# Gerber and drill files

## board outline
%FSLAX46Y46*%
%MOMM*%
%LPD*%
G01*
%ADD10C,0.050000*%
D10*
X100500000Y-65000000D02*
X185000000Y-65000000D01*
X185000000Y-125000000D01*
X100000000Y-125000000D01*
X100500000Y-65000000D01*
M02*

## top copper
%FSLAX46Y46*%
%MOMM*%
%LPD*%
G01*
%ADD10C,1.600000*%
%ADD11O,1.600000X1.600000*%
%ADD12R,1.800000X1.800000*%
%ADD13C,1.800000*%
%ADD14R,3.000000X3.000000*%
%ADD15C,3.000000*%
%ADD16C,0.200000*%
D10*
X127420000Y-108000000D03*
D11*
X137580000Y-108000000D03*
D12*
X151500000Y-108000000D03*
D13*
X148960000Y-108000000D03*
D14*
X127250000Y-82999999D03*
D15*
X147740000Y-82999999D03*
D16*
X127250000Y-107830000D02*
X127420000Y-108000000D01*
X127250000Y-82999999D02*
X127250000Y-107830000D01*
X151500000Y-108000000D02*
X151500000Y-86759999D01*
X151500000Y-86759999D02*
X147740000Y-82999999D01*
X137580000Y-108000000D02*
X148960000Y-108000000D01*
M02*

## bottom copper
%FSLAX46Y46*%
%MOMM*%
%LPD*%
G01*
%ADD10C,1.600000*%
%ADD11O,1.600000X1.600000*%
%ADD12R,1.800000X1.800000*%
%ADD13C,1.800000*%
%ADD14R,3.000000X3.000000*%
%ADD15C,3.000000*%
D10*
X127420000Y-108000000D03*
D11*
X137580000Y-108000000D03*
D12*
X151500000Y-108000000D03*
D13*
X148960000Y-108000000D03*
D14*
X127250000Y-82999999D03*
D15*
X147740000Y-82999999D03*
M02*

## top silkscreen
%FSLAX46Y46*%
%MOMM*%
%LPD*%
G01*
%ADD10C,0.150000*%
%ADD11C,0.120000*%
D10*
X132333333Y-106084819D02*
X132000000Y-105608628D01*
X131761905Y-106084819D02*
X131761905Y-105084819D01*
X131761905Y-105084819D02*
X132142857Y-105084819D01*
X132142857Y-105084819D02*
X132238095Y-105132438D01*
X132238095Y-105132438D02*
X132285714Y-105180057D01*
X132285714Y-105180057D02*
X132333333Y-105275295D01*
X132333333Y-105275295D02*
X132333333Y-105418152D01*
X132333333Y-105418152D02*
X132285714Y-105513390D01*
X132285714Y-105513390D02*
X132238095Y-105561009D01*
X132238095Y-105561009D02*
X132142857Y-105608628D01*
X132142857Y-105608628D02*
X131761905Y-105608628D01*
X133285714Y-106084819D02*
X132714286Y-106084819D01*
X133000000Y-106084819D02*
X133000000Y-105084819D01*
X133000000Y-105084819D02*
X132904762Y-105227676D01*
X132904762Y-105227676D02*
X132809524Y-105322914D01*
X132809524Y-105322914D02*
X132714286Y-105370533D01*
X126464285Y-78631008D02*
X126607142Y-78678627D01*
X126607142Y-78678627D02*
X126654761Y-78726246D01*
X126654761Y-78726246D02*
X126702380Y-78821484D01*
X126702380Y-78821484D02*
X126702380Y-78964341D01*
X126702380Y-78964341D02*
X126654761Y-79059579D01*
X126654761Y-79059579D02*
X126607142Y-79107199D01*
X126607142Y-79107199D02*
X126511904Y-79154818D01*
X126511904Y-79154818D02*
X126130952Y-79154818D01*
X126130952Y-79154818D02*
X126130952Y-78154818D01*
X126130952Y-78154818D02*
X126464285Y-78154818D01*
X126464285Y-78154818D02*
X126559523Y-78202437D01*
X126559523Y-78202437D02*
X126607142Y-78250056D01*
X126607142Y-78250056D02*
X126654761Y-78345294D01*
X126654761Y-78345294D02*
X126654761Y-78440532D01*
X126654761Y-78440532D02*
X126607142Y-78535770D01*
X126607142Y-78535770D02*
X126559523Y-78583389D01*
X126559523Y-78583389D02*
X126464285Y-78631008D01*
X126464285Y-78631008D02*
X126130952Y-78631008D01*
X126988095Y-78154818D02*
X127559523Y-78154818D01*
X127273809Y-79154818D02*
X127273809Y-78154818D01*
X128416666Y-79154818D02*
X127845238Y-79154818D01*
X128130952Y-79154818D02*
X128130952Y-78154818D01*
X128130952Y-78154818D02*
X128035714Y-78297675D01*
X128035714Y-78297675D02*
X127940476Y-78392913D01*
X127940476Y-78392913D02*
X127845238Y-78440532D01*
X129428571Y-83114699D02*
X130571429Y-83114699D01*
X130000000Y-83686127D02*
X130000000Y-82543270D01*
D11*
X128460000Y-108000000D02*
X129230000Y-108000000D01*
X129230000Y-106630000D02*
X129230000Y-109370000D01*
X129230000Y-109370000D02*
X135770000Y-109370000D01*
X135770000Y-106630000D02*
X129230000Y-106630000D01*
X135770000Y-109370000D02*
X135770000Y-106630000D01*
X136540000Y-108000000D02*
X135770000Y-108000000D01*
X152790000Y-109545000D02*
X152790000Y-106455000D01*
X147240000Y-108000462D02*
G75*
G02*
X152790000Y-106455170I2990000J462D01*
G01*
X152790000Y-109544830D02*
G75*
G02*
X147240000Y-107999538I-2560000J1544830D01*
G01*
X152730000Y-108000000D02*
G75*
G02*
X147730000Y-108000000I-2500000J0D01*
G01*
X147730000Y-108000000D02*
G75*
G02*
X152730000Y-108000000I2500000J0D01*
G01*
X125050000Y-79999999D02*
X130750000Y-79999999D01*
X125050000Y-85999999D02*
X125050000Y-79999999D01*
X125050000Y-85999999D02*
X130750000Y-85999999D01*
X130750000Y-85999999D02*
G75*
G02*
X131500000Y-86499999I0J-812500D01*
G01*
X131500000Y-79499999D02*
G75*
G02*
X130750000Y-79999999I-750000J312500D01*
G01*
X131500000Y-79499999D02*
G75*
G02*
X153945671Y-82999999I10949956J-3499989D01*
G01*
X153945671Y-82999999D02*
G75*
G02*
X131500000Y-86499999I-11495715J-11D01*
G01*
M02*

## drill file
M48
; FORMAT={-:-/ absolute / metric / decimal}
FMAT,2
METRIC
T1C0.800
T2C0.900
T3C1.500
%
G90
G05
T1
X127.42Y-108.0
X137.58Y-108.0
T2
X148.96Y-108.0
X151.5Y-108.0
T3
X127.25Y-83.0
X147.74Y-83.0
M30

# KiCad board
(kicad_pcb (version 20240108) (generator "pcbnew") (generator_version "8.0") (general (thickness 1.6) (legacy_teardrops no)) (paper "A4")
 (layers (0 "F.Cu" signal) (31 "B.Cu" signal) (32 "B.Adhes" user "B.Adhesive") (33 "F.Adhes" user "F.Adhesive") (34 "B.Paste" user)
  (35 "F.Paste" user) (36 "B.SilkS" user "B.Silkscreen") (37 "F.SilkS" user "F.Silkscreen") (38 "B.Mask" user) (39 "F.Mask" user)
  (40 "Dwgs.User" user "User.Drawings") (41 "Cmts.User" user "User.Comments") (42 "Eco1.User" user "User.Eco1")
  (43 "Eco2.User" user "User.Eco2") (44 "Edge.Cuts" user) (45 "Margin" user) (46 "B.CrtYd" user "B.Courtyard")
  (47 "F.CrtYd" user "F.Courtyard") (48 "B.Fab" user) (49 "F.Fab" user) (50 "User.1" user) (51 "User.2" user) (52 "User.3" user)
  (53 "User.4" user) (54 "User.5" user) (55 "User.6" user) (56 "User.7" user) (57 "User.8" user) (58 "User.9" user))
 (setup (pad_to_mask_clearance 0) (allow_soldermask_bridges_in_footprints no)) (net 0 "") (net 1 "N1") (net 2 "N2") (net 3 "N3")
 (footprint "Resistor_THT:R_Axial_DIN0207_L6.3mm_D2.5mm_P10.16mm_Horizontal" (layer "F.Cu") (at 127.42 108)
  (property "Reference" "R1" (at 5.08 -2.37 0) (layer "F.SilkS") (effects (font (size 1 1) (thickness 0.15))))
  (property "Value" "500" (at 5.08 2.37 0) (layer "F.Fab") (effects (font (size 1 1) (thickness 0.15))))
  (fp_line (start 1.04 0) (end 1.81 0) (stroke (width 0.12) (type solid)) (layer "F.SilkS"))
  (fp_line (start 1.81 -1.37) (end 1.81 1.37) (stroke (width 0.12) (type solid)) (layer "F.SilkS"))
  (fp_line (start 1.81 1.37) (end 8.35 1.37) (stroke (width 0.12) (type solid)) (layer "F.SilkS"))
  (fp_line (start 8.35 -1.37) (end 1.81 -1.37) (stroke (width 0.12) (type solid)) (layer "F.SilkS"))
  (fp_line (start 8.35 1.37) (end 8.35 -1.37) (stroke (width 0.12) (type solid)) (layer "F.SilkS"))
  (fp_line (start 9.12 0) (end 8.35 0) (stroke (width 0.12) (type solid)) (layer "F.SilkS"))
  (pad "1" thru_hole circle (at 0 0) (size 1.6 1.6) (drill 0.8) (layers "*.Cu" "*.Mask") (remove_unused_layers no) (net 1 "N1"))
  (pad "2" thru_hole oval (at 10.16 0) (size 1.6 1.6) (drill 0.8) (layers "*.Cu" "*.Mask") (remove_unused_layers no) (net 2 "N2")))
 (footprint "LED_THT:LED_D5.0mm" (layer "F.Cu") (at 151.5 108 180)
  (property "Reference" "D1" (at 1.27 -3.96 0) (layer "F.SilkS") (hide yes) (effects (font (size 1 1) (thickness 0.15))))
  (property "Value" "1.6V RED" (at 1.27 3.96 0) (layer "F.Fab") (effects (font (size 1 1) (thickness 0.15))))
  (fp_line (start -1.29 -1.545) (end -1.29 1.545) (stroke (width 0.12) (type solid)) (layer "F.SilkS"))
  (fp_arc (start 4.26 -0.000462) (mid 2.072002 2.880433) (end -1.29 1.54483) (stroke (width 0.12) (type solid)) (layer "F.SilkS"))
  (fp_arc (start -1.29 -1.54483) (mid 2.072002 -2.880433) (end 4.26 0.000462) (stroke (width 0.12) (type solid)) (layer "F.SilkS"))
  (fp_circle (center 1.27 0) (end 3.77 0) (stroke (width 0.12) (type solid)) (fill none) (layer "F.SilkS"))
  (pad "1" thru_hole rect (at 0 0 180) (size 1.8 1.8) (drill 0.9) (layers "*.Cu" "*.Mask") (remove_unused_layers no) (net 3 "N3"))
  (pad "2" thru_hole circle (at 2.54 0 180) (size 1.8 1.8) (drill 0.9) (layers "*.Cu" "*.Mask") (remove_unused_layers no) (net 2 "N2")))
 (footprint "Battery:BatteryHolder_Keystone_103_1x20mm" (layer "F.Cu") (at 127.25 82.999999)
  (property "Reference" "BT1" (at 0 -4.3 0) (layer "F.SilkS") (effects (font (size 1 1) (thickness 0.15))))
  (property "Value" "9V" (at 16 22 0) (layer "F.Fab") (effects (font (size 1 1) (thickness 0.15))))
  (fp_line (start -2.2 -3) (end 3.5 -3) (stroke (width 0.12) (type solid)) (layer "F.SilkS"))
  (fp_line (start -2.2 3) (end -2.2 -3) (stroke (width 0.12) (type solid)) (layer "F.SilkS"))
  (fp_line (start -2.2 3) (end 3.5 3) (stroke (width 0.12) (type solid)) (layer "F.SilkS"))
  (fp_arc (start 3.5 3) (mid 3.950694 3.136459) (end 4.25 3.5) (stroke (width 0.12) (type solid)) (layer "F.SilkS"))
  (fp_arc (start 4.25 -3.5) (mid 3.950694 -3.136459) (end 3.5 -3) (stroke (width 0.12) (type solid)) (layer "F.SilkS"))
  (fp_arc (start 4.25 -3.5) (mid 16.971103 -11.358466) (end 26.695671 0) (stroke (width 0.12) (type solid)) (layer "F.SilkS"))
  (fp_arc (start 26.695671 0) (mid 16.971103 11.358466) (end 4.25 3.5) (stroke (width 0.12) (type solid)) (layer "F.SilkS"))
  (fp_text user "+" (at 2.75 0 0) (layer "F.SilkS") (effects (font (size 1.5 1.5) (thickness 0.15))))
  (pad "1" thru_hole rect (at 0 0) (size 3 3) (drill 1.5) (layers "*.Cu" "*.Mask") (remove_unused_layers no) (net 1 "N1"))
  (pad "2" thru_hole circle (at 20.49 0) (size 3 3) (drill 1.5) (layers "*.Cu" "*.Mask") (remove_unused_layers no) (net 3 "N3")))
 (gr_poly (pts (xy 100.5 65) (xy 185 65) (xy 185 125) (xy 100 125)) (stroke (width 0.05) (type solid)) (fill none) (layer "Edge.Cuts"))
 (segment (start 127.25 107.83) (end 127.42 108) (width 0.2) (layer "F.Cu") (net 1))
 (segment (start 127.25 82.999999) (end 127.25 107.83) (width 0.2) (layer "F.Cu") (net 1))
 (segment (start 151.5 108) (end 151.5 86.759999) (width 0.2) (layer "F.Cu") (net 3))
 (segment (start 151.5 86.759999) (end 147.74 82.999999) (width 0.2) (layer "F.Cu") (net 3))
 (segment (start 137.58 108) (end 148.96 108) (width 0.2) (layer "F.Cu") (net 2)))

